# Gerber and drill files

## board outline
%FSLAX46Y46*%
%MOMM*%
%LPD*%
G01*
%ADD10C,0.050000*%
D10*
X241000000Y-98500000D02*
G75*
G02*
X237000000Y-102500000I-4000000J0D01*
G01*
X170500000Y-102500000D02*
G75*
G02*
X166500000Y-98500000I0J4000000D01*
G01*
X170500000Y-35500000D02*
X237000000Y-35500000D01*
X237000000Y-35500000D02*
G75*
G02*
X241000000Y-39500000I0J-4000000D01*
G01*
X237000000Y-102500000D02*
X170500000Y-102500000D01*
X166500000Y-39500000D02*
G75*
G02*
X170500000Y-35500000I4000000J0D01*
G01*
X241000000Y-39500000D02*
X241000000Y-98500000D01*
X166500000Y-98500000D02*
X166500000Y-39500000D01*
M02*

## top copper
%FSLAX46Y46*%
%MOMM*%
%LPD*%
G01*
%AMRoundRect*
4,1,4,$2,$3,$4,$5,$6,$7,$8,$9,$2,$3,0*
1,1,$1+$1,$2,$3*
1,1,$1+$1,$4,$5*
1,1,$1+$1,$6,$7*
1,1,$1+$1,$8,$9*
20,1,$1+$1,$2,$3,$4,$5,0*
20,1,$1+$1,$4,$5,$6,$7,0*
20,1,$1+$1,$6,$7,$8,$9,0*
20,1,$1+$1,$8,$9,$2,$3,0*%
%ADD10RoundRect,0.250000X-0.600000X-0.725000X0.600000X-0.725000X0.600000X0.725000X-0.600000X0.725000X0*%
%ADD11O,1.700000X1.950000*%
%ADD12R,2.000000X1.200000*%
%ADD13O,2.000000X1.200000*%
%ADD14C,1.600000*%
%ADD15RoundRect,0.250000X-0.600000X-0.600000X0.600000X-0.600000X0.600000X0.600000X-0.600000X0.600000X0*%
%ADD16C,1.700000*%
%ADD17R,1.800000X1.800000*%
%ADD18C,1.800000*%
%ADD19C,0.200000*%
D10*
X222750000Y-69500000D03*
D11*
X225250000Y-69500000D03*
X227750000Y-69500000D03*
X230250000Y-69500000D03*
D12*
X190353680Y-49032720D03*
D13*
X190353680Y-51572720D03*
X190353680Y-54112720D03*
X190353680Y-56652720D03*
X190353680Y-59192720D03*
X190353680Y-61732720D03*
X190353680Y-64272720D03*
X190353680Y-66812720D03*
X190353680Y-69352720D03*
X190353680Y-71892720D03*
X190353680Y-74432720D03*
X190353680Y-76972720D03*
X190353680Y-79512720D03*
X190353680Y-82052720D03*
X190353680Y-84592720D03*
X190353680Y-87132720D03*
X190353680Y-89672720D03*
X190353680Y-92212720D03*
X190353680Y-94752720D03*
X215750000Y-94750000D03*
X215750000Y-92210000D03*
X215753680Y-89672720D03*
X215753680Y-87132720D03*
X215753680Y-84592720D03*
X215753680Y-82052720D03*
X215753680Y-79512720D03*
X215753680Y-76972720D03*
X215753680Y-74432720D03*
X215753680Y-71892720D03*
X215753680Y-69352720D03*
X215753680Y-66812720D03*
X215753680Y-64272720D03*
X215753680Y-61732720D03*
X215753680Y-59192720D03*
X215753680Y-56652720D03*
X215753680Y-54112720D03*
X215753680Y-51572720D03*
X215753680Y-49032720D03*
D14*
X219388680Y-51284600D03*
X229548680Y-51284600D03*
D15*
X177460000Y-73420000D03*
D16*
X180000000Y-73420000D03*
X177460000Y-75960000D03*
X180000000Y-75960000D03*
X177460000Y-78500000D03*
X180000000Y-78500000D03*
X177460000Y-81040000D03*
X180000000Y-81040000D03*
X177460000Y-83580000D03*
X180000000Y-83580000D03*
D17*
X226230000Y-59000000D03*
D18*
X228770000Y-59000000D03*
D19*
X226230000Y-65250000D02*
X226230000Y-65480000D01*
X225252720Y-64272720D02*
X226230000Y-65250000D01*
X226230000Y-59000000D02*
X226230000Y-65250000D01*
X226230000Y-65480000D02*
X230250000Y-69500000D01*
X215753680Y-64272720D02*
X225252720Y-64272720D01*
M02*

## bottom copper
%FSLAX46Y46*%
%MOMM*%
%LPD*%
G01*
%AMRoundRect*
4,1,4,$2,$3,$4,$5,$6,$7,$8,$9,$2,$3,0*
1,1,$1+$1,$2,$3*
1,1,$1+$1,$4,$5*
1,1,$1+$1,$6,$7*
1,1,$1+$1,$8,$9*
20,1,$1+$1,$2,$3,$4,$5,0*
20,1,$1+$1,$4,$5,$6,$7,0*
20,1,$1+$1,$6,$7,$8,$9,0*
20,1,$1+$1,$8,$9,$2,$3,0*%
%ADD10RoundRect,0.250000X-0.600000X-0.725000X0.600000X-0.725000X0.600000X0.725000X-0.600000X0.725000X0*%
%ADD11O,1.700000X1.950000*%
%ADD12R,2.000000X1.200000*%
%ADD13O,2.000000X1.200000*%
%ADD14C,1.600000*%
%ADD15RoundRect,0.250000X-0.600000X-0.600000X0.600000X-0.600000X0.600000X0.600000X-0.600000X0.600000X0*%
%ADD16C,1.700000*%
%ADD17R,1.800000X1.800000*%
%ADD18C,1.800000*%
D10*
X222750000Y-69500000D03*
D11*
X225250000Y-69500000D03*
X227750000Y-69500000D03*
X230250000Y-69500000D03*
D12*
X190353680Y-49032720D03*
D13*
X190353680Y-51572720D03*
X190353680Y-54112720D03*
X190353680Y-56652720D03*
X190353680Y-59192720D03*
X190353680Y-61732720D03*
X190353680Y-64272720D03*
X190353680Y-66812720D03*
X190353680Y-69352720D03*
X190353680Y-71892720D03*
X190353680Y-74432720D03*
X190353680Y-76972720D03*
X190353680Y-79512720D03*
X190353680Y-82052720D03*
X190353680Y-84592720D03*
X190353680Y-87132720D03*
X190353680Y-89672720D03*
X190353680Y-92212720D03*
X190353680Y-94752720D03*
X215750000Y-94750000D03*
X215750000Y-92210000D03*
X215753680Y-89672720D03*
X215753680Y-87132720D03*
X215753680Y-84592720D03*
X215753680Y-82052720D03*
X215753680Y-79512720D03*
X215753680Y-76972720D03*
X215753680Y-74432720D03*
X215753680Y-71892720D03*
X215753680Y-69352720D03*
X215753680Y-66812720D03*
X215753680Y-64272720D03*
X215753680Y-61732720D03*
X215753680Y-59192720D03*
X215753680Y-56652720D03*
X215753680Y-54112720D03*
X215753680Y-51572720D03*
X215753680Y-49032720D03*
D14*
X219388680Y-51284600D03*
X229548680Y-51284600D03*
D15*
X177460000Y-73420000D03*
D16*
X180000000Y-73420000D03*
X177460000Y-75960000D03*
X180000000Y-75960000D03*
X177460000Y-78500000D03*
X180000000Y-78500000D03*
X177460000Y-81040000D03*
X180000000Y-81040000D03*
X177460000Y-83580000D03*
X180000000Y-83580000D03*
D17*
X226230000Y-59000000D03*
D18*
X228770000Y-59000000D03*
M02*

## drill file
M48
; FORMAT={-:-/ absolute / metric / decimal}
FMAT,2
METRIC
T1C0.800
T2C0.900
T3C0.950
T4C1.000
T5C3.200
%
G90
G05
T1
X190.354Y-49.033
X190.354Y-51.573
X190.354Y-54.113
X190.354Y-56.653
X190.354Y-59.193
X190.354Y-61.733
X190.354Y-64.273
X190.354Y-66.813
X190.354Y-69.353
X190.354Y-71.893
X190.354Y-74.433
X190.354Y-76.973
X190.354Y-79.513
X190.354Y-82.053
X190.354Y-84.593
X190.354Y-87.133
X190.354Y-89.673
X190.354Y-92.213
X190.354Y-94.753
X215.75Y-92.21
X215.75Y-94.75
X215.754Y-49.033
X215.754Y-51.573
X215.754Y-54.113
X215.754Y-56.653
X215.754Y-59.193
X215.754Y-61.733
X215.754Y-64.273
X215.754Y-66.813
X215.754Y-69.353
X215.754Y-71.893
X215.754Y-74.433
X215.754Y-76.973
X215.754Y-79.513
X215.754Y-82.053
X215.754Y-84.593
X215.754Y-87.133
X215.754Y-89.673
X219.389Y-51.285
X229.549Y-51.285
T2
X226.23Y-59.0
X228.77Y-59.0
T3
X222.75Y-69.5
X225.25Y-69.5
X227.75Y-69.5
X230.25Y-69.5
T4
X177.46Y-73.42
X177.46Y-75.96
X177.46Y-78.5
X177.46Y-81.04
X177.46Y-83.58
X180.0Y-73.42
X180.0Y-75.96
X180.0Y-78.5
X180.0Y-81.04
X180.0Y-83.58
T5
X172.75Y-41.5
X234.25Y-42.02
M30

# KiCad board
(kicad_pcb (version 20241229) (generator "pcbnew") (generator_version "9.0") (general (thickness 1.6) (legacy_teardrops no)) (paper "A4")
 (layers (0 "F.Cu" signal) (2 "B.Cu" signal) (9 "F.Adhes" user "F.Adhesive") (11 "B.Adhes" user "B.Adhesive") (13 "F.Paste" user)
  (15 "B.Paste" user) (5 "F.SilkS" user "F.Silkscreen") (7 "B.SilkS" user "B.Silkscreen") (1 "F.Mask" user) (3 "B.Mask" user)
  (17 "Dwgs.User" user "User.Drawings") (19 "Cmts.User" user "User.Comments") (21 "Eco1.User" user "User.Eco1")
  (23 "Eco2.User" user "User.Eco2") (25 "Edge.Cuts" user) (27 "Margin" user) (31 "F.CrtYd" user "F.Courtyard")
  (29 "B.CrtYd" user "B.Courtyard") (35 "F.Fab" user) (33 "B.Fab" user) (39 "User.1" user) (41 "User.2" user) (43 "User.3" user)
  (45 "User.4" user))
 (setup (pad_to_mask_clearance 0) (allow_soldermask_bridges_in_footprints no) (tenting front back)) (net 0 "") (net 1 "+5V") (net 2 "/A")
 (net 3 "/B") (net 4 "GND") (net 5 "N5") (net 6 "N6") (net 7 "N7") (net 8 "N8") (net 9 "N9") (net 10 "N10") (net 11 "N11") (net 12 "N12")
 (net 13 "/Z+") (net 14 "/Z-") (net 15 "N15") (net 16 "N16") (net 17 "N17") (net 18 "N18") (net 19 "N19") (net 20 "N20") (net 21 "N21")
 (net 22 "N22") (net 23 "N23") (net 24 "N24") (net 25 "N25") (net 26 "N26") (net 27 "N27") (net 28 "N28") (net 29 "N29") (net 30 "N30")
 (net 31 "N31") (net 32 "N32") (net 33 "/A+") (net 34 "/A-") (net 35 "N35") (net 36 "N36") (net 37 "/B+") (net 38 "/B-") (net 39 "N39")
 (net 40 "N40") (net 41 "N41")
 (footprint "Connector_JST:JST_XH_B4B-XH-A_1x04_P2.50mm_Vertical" (layer "F.Cu") (at 222.75 69.5)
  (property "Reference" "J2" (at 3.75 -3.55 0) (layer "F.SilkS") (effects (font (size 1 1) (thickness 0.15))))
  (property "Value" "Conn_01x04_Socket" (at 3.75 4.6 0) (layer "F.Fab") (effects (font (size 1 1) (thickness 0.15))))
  (pad "1" thru_hole roundrect (at 0 0) (size 1.7 1.95) (drill 0.95) (layers "*.Cu" "*.Mask") (remove_unused_layers no)
   (roundrect_rratio 0.147059) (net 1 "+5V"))
  (pad "2" thru_hole oval (at 2.5 0) (size 1.7 1.95) (drill 0.95) (layers "*.Cu" "*.Mask") (remove_unused_layers no) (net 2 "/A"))
  (pad "3" thru_hole oval (at 5 0) (size 1.7 1.95) (drill 0.95) (layers "*.Cu" "*.Mask") (remove_unused_layers no) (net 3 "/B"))
  (pad "4" thru_hole oval (at 7.5 0) (size 1.7 1.95) (drill 0.95) (layers "*.Cu" "*.Mask") (remove_unused_layers no) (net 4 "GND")))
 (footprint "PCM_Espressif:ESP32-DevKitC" (layer "F.Cu") (at 190.35368 49.03272)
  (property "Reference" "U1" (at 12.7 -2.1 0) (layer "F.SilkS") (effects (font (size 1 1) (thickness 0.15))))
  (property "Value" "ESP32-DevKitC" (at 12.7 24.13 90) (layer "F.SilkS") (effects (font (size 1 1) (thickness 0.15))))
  (pad "1" thru_hole rect (at 0 0 270) (size 1.2 2) (drill 0.8) (layers "*.Cu" "*.Mask") (remove_unused_layers no) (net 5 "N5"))
  (pad "2" thru_hole oval (at 0 2.54 270) (size 1.2 2) (drill 0.8) (layers "*.Cu" "*.Mask") (remove_unused_layers no) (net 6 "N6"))
  (pad "3" thru_hole oval (at 0 5.08 270) (size 1.2 2) (drill 0.8) (layers "*.Cu" "*.Mask") (remove_unused_layers no) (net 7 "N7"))
  (pad "4" thru_hole oval (at 0 7.62 270) (size 1.2 2) (drill 0.8) (layers "*.Cu" "*.Mask") (remove_unused_layers no) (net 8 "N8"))
  (pad "5" thru_hole oval (at 0 10.16 270) (size 1.2 2) (drill 0.8) (layers "*.Cu" "*.Mask") (remove_unused_layers no) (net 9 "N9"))
  (pad "6" thru_hole oval (at 0 12.7 270) (size 1.2 2) (drill 0.8) (layers "*.Cu" "*.Mask") (remove_unused_layers no) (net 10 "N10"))
  (pad "7" thru_hole oval (at 0 15.24 270) (size 1.2 2) (drill 0.8) (layers "*.Cu" "*.Mask") (remove_unused_layers no) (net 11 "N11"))
  (pad "8" thru_hole oval (at 0 17.78 270) (size 1.2 2) (drill 0.8) (layers "*.Cu" "*.Mask") (remove_unused_layers no) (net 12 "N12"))
  (pad "9" thru_hole oval (at 0 20.32 270) (size 1.2 2) (drill 0.8) (layers "*.Cu" "*.Mask") (remove_unused_layers no) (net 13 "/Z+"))
  (pad "10" thru_hole oval (at 0 22.86 270) (size 1.2 2) (drill 0.8) (layers "*.Cu" "*.Mask") (remove_unused_layers no) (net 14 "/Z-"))
  (pad "11" thru_hole oval (at 0 25.4 270) (size 1.2 2) (drill 0.8) (layers "*.Cu" "*.Mask") (remove_unused_layers no) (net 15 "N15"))
  (pad "12" thru_hole oval (at 0 27.94 270) (size 1.2 2) (drill 0.8) (layers "*.Cu" "*.Mask") (remove_unused_layers no) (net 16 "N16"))
  (pad "13" thru_hole oval (at 0 30.48 270) (size 1.2 2) (drill 0.8) (layers "*.Cu" "*.Mask") (remove_unused_layers no) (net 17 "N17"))
  (pad "14" thru_hole oval (at 0 33.02 270) (size 1.2 2) (drill 0.8) (layers "*.Cu" "*.Mask") (remove_unused_layers no) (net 4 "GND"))
  (pad "15" thru_hole oval (at 0 35.56 270) (size 1.2 2) (drill 0.8) (layers "*.Cu" "*.Mask") (remove_unused_layers no) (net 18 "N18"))
  (pad "16" thru_hole oval (at 0 38.1 270) (size 1.2 2) (drill 0.8) (layers "*.Cu" "*.Mask") (remove_unused_layers no) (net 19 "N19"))
  (pad "17" thru_hole oval (at 0 40.64 270) (size 1.2 2) (drill 0.8) (layers "*.Cu" "*.Mask") (remove_unused_layers no) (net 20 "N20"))
  (pad "18" thru_hole oval (at 0 43.18 270) (size 1.2 2) (drill 0.8) (layers "*.Cu" "*.Mask") (remove_unused_layers no) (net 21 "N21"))
  (pad "19" thru_hole oval (at 0 45.72 270) (size 1.2 2) (drill 0.8) (layers "*.Cu" "*.Mask") (remove_unused_layers no) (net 1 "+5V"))
  (pad "20" thru_hole oval (at 25.39632 45.71728 270) (size 1.2 2) (drill 0.8) (layers "*.Cu" "*.Mask") (remove_unused_layers no)
   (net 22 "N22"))
  (pad "21" thru_hole oval (at 25.39632 43.17728 270) (size 1.2 2) (drill 0.8) (layers "*.Cu" "*.Mask") (remove_unused_layers no)
   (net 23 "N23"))
  (pad "22" thru_hole oval (at 25.4 40.64 270) (size 1.2 2) (drill 0.8) (layers "*.Cu" "*.Mask") (remove_unused_layers no) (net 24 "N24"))
  (pad "23" thru_hole oval (at 25.4 38.1 270) (size 1.2 2) (drill 0.8) (layers "*.Cu" "*.Mask") (remove_unused_layers no) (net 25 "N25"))
  (pad "24" thru_hole oval (at 25.4 35.56 270) (size 1.2 2) (drill 0.8) (layers "*.Cu" "*.Mask") (remove_unused_layers no) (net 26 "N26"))
  (pad "25" thru_hole oval (at 25.4 33.02 270) (size 1.2 2) (drill 0.8) (layers "*.Cu" "*.Mask") (remove_unused_layers no) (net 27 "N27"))
  (pad "26" thru_hole oval (at 25.4 30.48 270) (size 1.2 2) (drill 0.8) (layers "*.Cu" "*.Mask") (remove_unused_layers no) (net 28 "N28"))
  (pad "27" thru_hole oval (at 25.4 27.94 270) (size 1.2 2) (drill 0.8) (layers "*.Cu" "*.Mask") (remove_unused_layers no) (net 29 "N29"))
  (pad "28" thru_hole oval (at 25.4 25.4 270) (size 1.2 2) (drill 0.8) (layers "*.Cu" "*.Mask") (remove_unused_layers no) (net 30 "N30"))
  (pad "29" thru_hole oval (at 25.4 22.86 270) (size 1.2 2) (drill 0.8) (layers "*.Cu" "*.Mask") (remove_unused_layers no) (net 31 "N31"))
  (pad "30" thru_hole oval (at 25.4 20.32 270) (size 1.2 2) (drill 0.8) (layers "*.Cu" "*.Mask") (remove_unused_layers no) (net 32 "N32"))
  (pad "31" thru_hole oval (at 25.4 17.78 270) (size 1.2 2) (drill 0.8) (layers "*.Cu" "*.Mask") (remove_unused_layers no) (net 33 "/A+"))
  (pad "32" thru_hole oval (at 25.4 15.24 270) (size 1.2 2) (drill 0.8) (layers "*.Cu" "*.Mask") (remove_unused_layers no) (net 4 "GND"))
  (pad "33" thru_hole oval (at 25.4 12.7 270) (size 1.2 2) (drill 0.8) (layers "*.Cu" "*.Mask") (remove_unused_layers no) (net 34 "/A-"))
  (pad "34" thru_hole oval (at 25.4 10.16 270) (size 1.2 2) (drill 0.8) (layers "*.Cu" "*.Mask") (remove_unused_layers no) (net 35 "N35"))
  (pad "35" thru_hole oval (at 25.4 7.62 270) (size 1.2 2) (drill 0.8) (layers "*.Cu" "*.Mask") (remove_unused_layers no) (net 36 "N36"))
  (pad "36" thru_hole oval (at 25.4 5.08 270) (size 1.2 2) (drill 0.8) (layers "*.Cu" "*.Mask") (remove_unused_layers no) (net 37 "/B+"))
  (pad "37" thru_hole oval (at 25.4 2.54 270) (size 1.2 2) (drill 0.8) (layers "*.Cu" "*.Mask") (remove_unused_layers no) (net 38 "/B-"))
  (pad "38" thru_hole oval (at 25.4 0 270) (size 1.2 2) (drill 0.8) (layers "*.Cu" "*.Mask") (remove_unused_layers no) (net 4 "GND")))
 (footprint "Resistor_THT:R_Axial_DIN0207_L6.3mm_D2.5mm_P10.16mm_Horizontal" (layer "F.Cu") (at 219.38868 51.2846)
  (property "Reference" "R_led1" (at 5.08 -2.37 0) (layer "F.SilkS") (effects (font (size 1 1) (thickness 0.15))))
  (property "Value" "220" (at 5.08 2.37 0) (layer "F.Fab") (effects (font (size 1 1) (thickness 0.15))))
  (pad "1" thru_hole circle (at 0 0) (size 1.6 1.6) (drill 0.8) (layers "*.Cu" "*.Mask") (remove_unused_layers no) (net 1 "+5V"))
  (pad "2" thru_hole circle (at 10.16 0) (size 1.6 1.6) (drill 0.8) (layers "*.Cu" "*.Mask") (remove_unused_layers no) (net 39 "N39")))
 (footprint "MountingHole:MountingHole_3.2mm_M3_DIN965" (layer "F.Cu") (at 234.25 42.0196)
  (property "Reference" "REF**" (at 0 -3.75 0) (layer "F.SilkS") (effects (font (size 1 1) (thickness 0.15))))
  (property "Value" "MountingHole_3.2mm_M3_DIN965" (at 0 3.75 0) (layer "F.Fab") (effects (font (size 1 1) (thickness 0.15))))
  (pad "" np_thru_hole circle (at 0 0) (size 3.2 3.2) (drill 3.2) (layers "*.Cu" "*.Mask")))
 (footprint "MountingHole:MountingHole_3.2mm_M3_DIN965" (layer "F.Cu") (at 172.75 41.5)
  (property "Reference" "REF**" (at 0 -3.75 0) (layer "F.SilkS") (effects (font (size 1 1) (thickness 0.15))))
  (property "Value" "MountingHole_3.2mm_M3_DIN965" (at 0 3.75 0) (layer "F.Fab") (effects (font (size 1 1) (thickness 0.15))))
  (pad "" np_thru_hole circle (at 0 0) (size 3.2 3.2) (drill 3.2) (layers "*.Cu" "*.Mask")))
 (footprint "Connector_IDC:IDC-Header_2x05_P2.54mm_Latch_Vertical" (layer "F.Cu") (at 177.46 73.42)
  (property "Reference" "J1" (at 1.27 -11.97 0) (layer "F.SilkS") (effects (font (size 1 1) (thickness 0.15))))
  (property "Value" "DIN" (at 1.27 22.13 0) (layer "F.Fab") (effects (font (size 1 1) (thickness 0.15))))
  (pad "1" thru_hole roundrect (at 0 0) (size 1.7 1.7) (drill 1) (layers "*.Cu" "*.Mask") (remove_unused_layers no)
   (roundrect_rratio 0.147059) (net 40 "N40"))
  (pad "2" thru_hole circle (at 2.54 0) (size 1.7 1.7) (drill 1) (layers "*.Cu" "*.Mask") (remove_unused_layers no) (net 1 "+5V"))
  (pad "3" thru_hole circle (at 0 2.54) (size 1.7 1.7) (drill 1) (layers "*.Cu" "*.Mask") (remove_unused_layers no) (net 4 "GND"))
  (pad "4" thru_hole circle (at 2.54 2.54) (size 1.7 1.7) (drill 1) (layers "*.Cu" "*.Mask") (remove_unused_layers no) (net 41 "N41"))
  (pad "5" thru_hole circle (at 0 5.08) (size 1.7 1.7) (drill 1) (layers "*.Cu" "*.Mask") (remove_unused_layers no) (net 34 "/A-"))
  (pad "6" thru_hole circle (at 2.54 5.08) (size 1.7 1.7) (drill 1) (layers "*.Cu" "*.Mask") (remove_unused_layers no) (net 33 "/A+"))
  (pad "7" thru_hole circle (at 0 7.62) (size 1.7 1.7) (drill 1) (layers "*.Cu" "*.Mask") (remove_unused_layers no) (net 38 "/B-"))
  (pad "8" thru_hole circle (at 2.54 7.62) (size 1.7 1.7) (drill 1) (layers "*.Cu" "*.Mask") (remove_unused_layers no) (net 37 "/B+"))
  (pad "9" thru_hole circle (at 0 10.16) (size 1.7 1.7) (drill 1) (layers "*.Cu" "*.Mask") (remove_unused_layers no) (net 14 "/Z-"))
  (pad "10" thru_hole circle (at 2.54 10.16) (size 1.7 1.7) (drill 1) (layers "*.Cu" "*.Mask") (remove_unused_layers no) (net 13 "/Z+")))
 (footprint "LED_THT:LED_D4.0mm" (layer "F.Cu") (at 226.23 59)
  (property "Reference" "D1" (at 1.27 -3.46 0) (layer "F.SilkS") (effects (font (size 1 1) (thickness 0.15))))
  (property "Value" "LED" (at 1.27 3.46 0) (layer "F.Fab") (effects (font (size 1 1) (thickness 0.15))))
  (pad "1" thru_hole rect (at 0 0) (size 1.8 1.8) (drill 0.9) (layers "*.Cu" "*.Mask") (remove_unused_layers no) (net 4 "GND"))
  (pad "2" thru_hole circle (at 2.54 0) (size 1.8 1.8) (drill 0.9) (layers "*.Cu" "*.Mask") (remove_unused_layers no) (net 39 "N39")))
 (gr_arc (start 241 98.5) (mid 239.828427 101.328427) (end 237 102.5) (stroke (width 0.05) (type default)) (layer "Edge.Cuts"))
 (gr_arc (start 170.5 102.5) (mid 167.671573 101.328427) (end 166.5 98.5) (stroke (width 0.05) (type default)) (layer "Edge.Cuts"))
 (gr_line (start 170.5 35.5) (end 237 35.5) (stroke (width 0.05) (type default)) (layer "Edge.Cuts"))
 (gr_arc (start 237 35.5) (mid 239.828427 36.671573) (end 241 39.5) (stroke (width 0.05) (type default)) (layer "Edge.Cuts"))
 (gr_line (start 237 102.5) (end 170.5 102.5) (stroke (width 0.05) (type default)) (layer "Edge.Cuts"))
 (gr_arc (start 166.5 39.5) (mid 167.671573 36.671573) (end 170.5 35.5) (stroke (width 0.05) (type default)) (layer "Edge.Cuts"))
 (gr_line (start 241 39.5) (end 241 98.5) (stroke (width 0.05) (type default)) (layer "Edge.Cuts"))
 (gr_line (start 166.5 98.5) (end 166.5 39.5) (stroke (width 0.05) (type default)) (layer "Edge.Cuts"))
 (segment (start 226.23 65.25) (end 226.23 65.48) (width 0.2) (layer "F.Cu") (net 4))
 (segment (start 225.25272 64.27272) (end 226.23 65.25) (width 0.2) (layer "F.Cu") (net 4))
 (segment (start 226.23 59) (end 226.23 65.25) (width 0.2) (layer "F.Cu") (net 4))
 (segment (start 226.23 65.48) (end 230.25 69.5) (width 0.2) (layer "F.Cu") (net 4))
 (segment (start 215.75368 64.27272) (end 225.25272 64.27272) (width 0.2) (layer "F.Cu") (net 4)))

